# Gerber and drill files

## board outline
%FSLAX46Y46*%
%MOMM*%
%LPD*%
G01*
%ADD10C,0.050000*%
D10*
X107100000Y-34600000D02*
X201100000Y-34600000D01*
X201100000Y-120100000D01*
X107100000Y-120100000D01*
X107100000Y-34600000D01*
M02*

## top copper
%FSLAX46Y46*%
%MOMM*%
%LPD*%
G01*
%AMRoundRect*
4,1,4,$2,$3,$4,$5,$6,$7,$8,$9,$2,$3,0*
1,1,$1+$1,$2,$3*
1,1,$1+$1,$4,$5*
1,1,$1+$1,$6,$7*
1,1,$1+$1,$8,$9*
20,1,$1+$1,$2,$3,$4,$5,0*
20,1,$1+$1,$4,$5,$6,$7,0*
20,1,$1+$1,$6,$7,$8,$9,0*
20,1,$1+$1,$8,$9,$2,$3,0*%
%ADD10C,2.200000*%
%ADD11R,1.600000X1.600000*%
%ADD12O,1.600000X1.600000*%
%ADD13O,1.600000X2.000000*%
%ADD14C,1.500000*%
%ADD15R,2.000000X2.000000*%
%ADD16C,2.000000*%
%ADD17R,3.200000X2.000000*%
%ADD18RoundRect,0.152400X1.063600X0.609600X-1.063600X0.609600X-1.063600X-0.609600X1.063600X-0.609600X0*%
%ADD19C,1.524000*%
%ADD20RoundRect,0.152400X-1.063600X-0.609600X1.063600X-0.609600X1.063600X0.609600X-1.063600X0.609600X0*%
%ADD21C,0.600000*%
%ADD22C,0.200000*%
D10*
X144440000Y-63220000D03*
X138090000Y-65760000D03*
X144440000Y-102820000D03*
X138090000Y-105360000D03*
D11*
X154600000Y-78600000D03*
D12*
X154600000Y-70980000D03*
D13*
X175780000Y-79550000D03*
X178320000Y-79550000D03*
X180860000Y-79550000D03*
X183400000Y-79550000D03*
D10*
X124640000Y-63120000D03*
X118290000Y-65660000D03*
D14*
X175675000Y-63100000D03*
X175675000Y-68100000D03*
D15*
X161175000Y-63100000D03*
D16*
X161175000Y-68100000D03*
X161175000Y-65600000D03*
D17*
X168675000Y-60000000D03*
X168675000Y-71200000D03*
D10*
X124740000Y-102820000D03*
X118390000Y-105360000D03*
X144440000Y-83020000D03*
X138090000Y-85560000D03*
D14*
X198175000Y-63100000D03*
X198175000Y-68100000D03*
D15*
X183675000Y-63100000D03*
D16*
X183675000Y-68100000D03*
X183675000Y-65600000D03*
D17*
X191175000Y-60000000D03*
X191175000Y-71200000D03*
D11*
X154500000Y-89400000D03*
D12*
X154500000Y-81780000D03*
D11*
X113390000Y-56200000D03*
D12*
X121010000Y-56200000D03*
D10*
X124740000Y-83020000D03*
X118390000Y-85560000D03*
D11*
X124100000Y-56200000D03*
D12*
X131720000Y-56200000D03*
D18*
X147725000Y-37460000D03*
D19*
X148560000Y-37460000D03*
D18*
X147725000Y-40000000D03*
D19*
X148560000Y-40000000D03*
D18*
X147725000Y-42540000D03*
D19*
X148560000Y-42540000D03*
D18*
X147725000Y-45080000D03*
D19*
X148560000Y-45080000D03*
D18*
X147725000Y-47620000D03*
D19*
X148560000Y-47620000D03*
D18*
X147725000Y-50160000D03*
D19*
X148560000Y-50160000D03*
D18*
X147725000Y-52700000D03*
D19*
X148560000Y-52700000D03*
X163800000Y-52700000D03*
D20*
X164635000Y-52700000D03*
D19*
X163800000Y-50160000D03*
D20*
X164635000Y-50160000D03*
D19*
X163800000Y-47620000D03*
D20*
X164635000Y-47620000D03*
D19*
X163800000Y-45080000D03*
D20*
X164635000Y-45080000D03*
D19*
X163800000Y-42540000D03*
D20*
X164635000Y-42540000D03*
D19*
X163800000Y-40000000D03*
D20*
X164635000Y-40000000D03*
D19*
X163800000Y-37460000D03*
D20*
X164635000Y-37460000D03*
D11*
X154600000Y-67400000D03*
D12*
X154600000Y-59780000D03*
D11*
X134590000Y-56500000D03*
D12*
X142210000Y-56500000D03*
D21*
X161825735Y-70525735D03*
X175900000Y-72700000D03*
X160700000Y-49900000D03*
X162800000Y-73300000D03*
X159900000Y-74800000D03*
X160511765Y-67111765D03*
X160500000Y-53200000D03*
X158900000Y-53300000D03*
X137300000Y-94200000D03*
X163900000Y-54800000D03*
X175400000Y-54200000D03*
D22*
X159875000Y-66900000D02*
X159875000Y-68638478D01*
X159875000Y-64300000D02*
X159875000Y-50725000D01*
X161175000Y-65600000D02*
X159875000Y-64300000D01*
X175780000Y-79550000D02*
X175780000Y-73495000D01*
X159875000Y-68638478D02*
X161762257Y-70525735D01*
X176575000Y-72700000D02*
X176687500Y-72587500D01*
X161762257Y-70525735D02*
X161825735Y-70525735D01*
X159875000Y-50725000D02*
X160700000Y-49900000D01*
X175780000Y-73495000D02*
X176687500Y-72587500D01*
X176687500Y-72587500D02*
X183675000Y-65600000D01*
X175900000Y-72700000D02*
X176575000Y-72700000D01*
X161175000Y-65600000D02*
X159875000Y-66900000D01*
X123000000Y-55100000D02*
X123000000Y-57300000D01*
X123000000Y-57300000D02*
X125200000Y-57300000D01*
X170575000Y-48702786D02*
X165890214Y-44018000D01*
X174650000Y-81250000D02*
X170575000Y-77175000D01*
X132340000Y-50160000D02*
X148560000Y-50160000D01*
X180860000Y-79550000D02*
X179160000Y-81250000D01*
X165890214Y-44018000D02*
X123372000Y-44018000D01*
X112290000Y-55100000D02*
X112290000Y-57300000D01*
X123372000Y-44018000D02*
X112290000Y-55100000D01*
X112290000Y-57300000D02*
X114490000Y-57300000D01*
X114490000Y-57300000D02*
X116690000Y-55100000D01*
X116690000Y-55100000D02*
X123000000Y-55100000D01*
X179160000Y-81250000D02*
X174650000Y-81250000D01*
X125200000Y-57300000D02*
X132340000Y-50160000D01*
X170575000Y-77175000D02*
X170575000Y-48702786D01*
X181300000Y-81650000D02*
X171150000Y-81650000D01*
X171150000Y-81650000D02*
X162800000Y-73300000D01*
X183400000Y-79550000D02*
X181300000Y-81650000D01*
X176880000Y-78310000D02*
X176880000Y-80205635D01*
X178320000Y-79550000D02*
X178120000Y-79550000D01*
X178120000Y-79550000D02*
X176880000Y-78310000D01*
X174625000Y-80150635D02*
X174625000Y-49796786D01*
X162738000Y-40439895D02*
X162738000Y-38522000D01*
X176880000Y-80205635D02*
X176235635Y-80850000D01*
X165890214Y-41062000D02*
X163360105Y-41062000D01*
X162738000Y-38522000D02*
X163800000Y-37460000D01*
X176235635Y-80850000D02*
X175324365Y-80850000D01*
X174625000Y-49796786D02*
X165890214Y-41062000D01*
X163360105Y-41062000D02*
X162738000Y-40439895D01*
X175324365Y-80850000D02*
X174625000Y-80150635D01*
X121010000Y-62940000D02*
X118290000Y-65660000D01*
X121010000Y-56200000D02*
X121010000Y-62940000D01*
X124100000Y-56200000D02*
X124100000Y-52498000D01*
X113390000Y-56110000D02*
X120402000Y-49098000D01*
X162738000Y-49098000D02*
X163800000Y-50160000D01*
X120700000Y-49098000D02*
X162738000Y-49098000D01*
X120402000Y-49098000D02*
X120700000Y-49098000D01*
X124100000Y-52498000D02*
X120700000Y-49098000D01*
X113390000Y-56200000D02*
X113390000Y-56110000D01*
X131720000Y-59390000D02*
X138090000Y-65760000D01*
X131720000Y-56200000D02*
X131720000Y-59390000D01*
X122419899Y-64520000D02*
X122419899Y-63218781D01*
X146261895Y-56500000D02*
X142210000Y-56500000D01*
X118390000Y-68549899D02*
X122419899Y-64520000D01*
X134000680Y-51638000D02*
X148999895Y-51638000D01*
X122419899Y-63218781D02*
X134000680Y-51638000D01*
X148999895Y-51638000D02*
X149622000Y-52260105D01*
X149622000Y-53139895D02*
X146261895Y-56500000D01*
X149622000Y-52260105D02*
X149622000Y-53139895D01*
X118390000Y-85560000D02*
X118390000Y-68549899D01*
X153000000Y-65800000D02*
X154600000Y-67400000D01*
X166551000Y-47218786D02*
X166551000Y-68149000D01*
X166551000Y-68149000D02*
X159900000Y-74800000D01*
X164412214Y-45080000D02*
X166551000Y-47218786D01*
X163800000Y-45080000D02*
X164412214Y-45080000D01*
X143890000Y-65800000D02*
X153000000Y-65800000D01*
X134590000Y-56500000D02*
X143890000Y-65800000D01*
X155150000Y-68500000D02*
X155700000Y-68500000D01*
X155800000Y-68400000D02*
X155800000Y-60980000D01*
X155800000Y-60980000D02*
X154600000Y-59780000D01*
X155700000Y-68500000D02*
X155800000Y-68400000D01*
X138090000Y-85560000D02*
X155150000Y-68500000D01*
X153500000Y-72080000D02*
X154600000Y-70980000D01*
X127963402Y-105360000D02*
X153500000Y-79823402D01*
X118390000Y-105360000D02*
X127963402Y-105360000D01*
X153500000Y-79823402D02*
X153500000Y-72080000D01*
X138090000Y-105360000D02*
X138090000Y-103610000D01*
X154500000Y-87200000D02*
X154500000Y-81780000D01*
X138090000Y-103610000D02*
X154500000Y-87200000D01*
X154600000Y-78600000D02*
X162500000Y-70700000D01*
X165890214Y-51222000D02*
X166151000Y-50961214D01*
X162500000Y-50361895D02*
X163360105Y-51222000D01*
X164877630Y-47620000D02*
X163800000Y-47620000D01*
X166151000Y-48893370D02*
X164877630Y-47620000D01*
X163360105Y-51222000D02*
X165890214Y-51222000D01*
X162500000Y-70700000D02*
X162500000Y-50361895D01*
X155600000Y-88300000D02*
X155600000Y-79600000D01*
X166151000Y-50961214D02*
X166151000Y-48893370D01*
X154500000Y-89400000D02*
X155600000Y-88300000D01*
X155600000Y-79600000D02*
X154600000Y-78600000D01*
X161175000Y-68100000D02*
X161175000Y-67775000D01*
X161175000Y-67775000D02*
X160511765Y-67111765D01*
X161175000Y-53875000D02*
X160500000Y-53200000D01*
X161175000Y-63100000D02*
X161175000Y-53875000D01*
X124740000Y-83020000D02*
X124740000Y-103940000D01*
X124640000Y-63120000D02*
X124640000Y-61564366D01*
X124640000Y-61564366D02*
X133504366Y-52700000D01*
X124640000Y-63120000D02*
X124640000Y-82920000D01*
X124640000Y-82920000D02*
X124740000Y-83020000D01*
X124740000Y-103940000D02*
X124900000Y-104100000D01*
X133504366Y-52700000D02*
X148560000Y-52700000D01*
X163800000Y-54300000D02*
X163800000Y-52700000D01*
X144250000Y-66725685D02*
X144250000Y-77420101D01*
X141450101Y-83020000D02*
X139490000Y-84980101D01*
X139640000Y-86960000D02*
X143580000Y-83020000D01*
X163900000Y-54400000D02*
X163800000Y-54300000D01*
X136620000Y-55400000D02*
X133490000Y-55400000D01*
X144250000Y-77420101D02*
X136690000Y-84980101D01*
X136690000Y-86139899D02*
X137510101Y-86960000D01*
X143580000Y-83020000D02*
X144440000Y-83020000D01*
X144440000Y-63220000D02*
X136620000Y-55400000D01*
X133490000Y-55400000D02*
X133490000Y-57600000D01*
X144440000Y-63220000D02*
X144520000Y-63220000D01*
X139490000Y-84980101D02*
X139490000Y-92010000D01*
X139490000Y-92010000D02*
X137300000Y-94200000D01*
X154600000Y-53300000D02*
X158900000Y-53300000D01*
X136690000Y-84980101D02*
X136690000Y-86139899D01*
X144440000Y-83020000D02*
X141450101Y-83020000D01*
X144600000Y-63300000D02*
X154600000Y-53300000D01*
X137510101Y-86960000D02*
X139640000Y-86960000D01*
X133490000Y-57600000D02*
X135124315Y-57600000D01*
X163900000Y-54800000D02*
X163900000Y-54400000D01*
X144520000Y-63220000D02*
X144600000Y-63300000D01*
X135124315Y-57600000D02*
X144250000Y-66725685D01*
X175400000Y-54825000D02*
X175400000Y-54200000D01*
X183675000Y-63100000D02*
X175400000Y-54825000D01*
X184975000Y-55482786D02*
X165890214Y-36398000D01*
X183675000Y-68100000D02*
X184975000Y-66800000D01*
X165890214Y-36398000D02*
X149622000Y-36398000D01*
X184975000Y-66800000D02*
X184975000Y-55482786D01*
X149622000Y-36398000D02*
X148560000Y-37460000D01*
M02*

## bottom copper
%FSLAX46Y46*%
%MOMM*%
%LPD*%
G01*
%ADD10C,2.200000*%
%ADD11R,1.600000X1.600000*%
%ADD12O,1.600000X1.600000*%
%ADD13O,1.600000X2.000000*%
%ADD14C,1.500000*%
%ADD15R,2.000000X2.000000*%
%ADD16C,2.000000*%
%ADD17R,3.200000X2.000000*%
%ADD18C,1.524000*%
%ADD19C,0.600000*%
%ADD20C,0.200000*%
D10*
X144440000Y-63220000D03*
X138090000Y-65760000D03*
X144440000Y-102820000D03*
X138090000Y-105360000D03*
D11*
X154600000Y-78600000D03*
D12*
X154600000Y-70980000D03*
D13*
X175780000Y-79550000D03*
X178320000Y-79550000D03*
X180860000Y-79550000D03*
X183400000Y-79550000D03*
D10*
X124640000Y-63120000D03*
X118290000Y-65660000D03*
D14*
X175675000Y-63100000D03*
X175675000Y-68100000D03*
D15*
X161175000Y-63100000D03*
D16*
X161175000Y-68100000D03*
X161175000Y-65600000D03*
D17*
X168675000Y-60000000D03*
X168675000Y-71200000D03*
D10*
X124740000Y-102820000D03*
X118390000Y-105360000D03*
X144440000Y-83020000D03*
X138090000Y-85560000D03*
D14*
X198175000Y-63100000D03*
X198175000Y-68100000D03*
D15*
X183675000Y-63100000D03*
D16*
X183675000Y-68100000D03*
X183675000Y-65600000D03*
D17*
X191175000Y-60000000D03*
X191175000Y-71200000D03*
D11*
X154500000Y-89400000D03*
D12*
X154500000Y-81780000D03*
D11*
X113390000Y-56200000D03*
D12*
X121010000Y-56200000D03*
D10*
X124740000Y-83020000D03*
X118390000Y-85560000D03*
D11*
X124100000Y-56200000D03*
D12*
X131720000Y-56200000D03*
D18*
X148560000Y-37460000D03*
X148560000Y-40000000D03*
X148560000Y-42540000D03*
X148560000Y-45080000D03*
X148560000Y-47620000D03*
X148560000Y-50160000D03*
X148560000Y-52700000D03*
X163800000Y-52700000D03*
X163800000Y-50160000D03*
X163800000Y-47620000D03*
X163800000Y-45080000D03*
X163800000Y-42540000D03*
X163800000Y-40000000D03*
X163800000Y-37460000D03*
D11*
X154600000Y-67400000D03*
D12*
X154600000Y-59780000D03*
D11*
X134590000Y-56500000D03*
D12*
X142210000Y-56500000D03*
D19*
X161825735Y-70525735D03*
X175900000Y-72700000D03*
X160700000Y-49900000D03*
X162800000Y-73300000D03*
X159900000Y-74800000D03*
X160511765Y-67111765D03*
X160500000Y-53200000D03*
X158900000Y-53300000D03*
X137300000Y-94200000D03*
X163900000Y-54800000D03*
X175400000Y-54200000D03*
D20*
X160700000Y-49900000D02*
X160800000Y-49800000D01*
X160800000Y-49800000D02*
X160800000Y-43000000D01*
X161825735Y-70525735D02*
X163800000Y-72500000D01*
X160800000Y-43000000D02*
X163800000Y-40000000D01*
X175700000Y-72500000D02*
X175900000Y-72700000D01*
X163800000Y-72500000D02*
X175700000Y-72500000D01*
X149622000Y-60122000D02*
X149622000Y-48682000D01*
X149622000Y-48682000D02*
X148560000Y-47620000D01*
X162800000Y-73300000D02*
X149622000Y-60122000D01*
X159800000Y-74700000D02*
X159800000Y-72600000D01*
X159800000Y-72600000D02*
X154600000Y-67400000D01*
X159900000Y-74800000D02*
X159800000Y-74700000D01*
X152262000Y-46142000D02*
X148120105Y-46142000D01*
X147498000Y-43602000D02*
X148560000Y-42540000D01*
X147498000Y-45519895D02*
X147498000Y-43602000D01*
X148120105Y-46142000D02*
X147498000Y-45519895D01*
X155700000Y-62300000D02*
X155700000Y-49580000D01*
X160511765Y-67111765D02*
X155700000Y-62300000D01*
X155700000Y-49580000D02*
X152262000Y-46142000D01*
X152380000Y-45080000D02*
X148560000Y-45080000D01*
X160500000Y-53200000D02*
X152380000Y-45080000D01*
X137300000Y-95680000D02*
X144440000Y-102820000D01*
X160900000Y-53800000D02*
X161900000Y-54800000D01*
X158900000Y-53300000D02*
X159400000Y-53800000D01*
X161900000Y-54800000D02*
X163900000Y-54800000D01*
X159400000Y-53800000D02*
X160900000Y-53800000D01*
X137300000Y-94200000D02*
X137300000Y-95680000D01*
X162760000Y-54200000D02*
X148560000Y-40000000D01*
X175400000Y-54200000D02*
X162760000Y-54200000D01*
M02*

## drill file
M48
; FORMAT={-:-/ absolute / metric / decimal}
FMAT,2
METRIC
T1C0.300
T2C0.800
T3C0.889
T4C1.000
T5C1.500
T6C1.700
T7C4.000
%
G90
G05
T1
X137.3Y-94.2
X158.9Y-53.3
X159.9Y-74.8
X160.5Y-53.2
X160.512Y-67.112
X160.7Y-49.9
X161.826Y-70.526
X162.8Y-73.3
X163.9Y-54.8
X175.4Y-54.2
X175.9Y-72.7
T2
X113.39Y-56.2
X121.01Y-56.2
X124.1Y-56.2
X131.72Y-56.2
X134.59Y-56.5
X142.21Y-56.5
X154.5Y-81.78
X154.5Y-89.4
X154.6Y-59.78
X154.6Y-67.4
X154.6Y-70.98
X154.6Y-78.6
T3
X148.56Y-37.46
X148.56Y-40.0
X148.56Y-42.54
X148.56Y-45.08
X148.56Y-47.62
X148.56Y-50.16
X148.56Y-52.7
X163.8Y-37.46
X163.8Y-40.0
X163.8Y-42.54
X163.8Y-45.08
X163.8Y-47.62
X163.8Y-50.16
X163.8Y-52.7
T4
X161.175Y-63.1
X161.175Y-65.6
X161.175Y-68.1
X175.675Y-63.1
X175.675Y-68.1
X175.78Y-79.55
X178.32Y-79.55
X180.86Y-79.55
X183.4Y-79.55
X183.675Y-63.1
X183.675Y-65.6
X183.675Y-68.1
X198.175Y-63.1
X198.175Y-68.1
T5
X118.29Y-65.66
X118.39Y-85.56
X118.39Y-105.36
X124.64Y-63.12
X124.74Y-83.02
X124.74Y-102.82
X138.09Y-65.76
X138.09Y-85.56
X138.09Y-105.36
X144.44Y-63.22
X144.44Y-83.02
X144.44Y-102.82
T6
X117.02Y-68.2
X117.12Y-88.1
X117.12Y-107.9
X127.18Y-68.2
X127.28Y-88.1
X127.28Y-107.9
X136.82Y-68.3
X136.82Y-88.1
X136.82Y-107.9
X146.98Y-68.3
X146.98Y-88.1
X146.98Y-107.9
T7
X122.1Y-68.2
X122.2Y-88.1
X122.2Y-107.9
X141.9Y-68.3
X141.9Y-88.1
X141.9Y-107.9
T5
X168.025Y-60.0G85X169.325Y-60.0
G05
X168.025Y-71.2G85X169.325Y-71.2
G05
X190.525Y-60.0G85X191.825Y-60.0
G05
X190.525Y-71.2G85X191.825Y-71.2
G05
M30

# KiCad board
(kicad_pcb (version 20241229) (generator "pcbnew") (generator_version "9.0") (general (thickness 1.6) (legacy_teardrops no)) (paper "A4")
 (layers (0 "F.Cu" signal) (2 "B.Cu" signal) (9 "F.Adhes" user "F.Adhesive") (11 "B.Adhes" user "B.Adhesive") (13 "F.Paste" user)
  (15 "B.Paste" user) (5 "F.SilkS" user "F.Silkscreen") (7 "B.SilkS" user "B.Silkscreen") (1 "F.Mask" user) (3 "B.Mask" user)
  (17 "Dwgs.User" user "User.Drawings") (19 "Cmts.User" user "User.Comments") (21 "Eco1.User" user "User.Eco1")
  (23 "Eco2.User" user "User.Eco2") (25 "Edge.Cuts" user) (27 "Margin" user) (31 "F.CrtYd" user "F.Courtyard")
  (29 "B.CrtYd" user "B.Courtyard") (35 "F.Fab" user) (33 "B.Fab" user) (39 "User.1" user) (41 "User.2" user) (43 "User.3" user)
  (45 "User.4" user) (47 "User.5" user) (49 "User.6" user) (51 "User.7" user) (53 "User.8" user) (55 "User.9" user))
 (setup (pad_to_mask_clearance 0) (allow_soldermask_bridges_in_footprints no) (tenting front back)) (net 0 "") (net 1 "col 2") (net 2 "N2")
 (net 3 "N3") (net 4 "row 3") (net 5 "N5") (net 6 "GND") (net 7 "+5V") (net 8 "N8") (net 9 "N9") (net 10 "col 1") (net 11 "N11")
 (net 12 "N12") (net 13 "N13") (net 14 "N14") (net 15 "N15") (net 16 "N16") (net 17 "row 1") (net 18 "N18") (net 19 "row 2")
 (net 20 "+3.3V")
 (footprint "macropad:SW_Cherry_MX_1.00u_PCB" (layer "F.Cu") (at 144.44 63.22)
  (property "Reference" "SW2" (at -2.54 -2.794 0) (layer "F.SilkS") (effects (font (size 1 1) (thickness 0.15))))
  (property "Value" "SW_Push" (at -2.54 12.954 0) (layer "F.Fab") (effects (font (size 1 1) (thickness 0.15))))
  (pad "" np_thru_hole circle (at -7.62 5.08) (size 1.7 1.7) (drill 1.7) (layers "*.Cu" "*.Mask"))
  (pad "" np_thru_hole circle (at -2.54 5.08) (size 4 4) (drill 4) (layers "*.Cu" "*.Mask"))
  (pad "" np_thru_hole circle (at 2.54 5.08) (size 1.7 1.7) (drill 1.7) (layers "*.Cu" "*.Mask"))
  (pad "1" thru_hole circle (at 0 0) (size 2.2 2.2) (drill 1.5) (layers "*.Cu" "*.Mask") (remove_unused_layers no) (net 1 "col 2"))
  (pad "2" thru_hole circle (at -6.35 2.54) (size 2.2 2.2) (drill 1.5) (layers "*.Cu" "*.Mask") (remove_unused_layers no) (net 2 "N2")))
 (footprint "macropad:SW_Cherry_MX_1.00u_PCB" (layer "F.Cu") (at 144.44 102.82)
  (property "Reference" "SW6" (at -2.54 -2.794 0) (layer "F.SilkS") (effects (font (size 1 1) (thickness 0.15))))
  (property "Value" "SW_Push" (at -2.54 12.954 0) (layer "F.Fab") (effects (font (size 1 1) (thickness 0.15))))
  (pad "" np_thru_hole circle (at -7.62 5.08) (size 1.7 1.7) (drill 1.7) (layers "*.Cu" "*.Mask"))
  (pad "" np_thru_hole circle (at -2.54 5.08) (size 4 4) (drill 4) (layers "*.Cu" "*.Mask"))
  (pad "" np_thru_hole circle (at 2.54 5.08) (size 1.7 1.7) (drill 1.7) (layers "*.Cu" "*.Mask"))
  (pad "1" thru_hole circle (at 0 0) (size 2.2 2.2) (drill 1.5) (layers "*.Cu" "*.Mask") (remove_unused_layers no) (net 1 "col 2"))
  (pad "2" thru_hole circle (at -6.35 2.54) (size 2.2 2.2) (drill 1.5) (layers "*.Cu" "*.Mask") (remove_unused_layers no) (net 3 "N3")))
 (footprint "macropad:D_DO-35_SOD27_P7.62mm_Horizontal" (layer "F.Cu") (at 154.6 78.6 90)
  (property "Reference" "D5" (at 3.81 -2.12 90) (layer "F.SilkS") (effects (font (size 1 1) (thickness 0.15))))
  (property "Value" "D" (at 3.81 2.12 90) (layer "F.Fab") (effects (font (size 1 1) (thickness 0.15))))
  (pad "1" thru_hole rect (at 0 0 90) (size 1.6 1.6) (drill 0.8) (layers "*.Cu" "*.Mask") (remove_unused_layers no) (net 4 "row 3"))
  (pad "2" thru_hole oval (at 7.62 0 90) (size 1.6 1.6) (drill 0.8) (layers "*.Cu" "*.Mask") (remove_unused_layers no) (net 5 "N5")))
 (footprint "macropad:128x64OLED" (layer "F.Cu") (at 179.4 90.15)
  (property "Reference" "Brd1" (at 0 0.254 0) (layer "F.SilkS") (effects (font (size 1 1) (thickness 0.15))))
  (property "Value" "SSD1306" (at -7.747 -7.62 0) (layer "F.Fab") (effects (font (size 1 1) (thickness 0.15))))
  (pad "1" thru_hole oval (at -3.62 -10.6 90) (size 2 1.6) (drill 1) (layers "*.Cu" "*.Mask") (remove_unused_layers no) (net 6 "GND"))
  (pad "2" thru_hole oval (at -1.08 -10.6 90) (size 2 1.6) (drill 1) (layers "*.Cu" "*.Mask") (remove_unused_layers no) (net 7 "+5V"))
  (pad "3" thru_hole oval (at 1.46 -10.6 90) (size 2 1.6) (drill 1) (layers "*.Cu" "*.Mask") (remove_unused_layers no) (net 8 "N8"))
  (pad "4" thru_hole oval (at 4 -10.6 90) (size 2 1.6) (drill 1) (layers "*.Cu" "*.Mask") (remove_unused_layers no) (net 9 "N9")))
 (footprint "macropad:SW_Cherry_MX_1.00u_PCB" (layer "F.Cu") (at 124.64 63.12)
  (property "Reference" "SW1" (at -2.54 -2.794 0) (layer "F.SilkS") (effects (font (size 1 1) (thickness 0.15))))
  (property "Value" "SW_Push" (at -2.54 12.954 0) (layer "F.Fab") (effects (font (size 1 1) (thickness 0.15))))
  (pad "" np_thru_hole circle (at -7.62 5.08) (size 1.7 1.7) (drill 1.7) (layers "*.Cu" "*.Mask"))
  (pad "" np_thru_hole circle (at -2.54 5.08) (size 4 4) (drill 4) (layers "*.Cu" "*.Mask"))
  (pad "" np_thru_hole circle (at 2.54 5.08) (size 1.7 1.7) (drill 1.7) (layers "*.Cu" "*.Mask"))
  (pad "1" thru_hole circle (at 0 0) (size 2.2 2.2) (drill 1.5) (layers "*.Cu" "*.Mask") (remove_unused_layers no) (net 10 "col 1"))
  (pad "2" thru_hole circle (at -6.35 2.54) (size 2.2 2.2) (drill 1.5) (layers "*.Cu" "*.Mask") (remove_unused_layers no) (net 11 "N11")))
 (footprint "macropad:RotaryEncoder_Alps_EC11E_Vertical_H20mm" (layer "F.Cu") (at 161.175 63.1)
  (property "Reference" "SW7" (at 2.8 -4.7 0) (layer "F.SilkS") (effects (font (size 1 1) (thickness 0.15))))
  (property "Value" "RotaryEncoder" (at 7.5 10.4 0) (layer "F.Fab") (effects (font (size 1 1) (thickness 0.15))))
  (pad "" thru_hole circle (at 14.5 0) (size 1.5 1.5) (drill 1) (layers "*.Cu" "*.Mask") (remove_unused_layers no))
  (pad "" thru_hole circle (at 14.5 5) (size 1.5 1.5) (drill 1) (layers "*.Cu" "*.Mask") (remove_unused_layers no))
  (pad "A" thru_hole rect (at 0 0) (size 2 2) (drill 1) (layers "*.Cu" "*.Mask") (remove_unused_layers no) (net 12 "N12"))
  (pad "B" thru_hole circle (at 0 5) (size 2 2) (drill 1) (layers "*.Cu" "*.Mask") (remove_unused_layers no) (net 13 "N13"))
  (pad "C" thru_hole circle (at 0 2.5) (size 2 2) (drill 1) (layers "*.Cu" "*.Mask") (remove_unused_layers no) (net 6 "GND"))
  (pad "MP" thru_hole rect (at 7.5 -3.1) (size 3.2 2) (drill oval 2.8 1.5) (layers "*.Cu" "*.Mask") (remove_unused_layers no))
  (pad "MP" thru_hole rect (at 7.5 8.1) (size 3.2 2) (drill oval 2.8 1.5) (layers "*.Cu" "*.Mask") (remove_unused_layers no)))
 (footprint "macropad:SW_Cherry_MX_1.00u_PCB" (layer "F.Cu") (at 124.74 102.82)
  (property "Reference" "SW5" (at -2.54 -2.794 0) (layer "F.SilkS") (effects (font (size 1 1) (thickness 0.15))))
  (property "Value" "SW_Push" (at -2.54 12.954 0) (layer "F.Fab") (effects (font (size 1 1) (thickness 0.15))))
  (pad "" np_thru_hole circle (at -7.62 5.08) (size 1.7 1.7) (drill 1.7) (layers "*.Cu" "*.Mask"))
  (pad "" np_thru_hole circle (at -2.54 5.08) (size 4 4) (drill 4) (layers "*.Cu" "*.Mask"))
  (pad "" np_thru_hole circle (at 2.54 5.08) (size 1.7 1.7) (drill 1.7) (layers "*.Cu" "*.Mask"))
  (pad "1" thru_hole circle (at 0 0) (size 2.2 2.2) (drill 1.5) (layers "*.Cu" "*.Mask") (remove_unused_layers no) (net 10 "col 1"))
  (pad "2" thru_hole circle (at -6.35 2.54) (size 2.2 2.2) (drill 1.5) (layers "*.Cu" "*.Mask") (remove_unused_layers no) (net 5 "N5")))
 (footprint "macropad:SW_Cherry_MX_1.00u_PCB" (layer "F.Cu") (at 144.44 83.02)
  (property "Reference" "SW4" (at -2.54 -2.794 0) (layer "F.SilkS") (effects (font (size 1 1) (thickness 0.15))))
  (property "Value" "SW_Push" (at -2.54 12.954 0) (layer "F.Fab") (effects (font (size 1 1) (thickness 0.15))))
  (pad "" np_thru_hole circle (at -7.62 5.08) (size 1.7 1.7) (drill 1.7) (layers "*.Cu" "*.Mask"))
  (pad "" np_thru_hole circle (at -2.54 5.08) (size 4 4) (drill 4) (layers "*.Cu" "*.Mask"))
  (pad "" np_thru_hole circle (at 2.54 5.08) (size 1.7 1.7) (drill 1.7) (layers "*.Cu" "*.Mask"))
  (pad "1" thru_hole circle (at 0 0) (size 2.2 2.2) (drill 1.5) (layers "*.Cu" "*.Mask") (remove_unused_layers no) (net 1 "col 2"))
  (pad "2" thru_hole circle (at -6.35 2.54) (size 2.2 2.2) (drill 1.5) (layers "*.Cu" "*.Mask") (remove_unused_layers no) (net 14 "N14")))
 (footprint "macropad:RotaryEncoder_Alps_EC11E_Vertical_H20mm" (layer "F.Cu") (at 183.675 63.1)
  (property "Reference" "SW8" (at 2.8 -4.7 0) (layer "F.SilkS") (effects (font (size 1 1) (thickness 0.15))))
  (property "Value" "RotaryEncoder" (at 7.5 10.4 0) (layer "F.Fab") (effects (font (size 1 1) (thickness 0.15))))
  (pad "" thru_hole circle (at 14.5 0) (size 1.5 1.5) (drill 1) (layers "*.Cu" "*.Mask") (remove_unused_layers no))
  (pad "" thru_hole circle (at 14.5 5) (size 1.5 1.5) (drill 1) (layers "*.Cu" "*.Mask") (remove_unused_layers no))
  (pad "A" thru_hole rect (at 0 0) (size 2 2) (drill 1) (layers "*.Cu" "*.Mask") (remove_unused_layers no) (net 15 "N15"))
  (pad "B" thru_hole circle (at 0 5) (size 2 2) (drill 1) (layers "*.Cu" "*.Mask") (remove_unused_layers no) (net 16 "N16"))
  (pad "C" thru_hole circle (at 0 2.5) (size 2 2) (drill 1) (layers "*.Cu" "*.Mask") (remove_unused_layers no) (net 6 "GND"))
  (pad "MP" thru_hole rect (at 7.5 -3.1) (size 3.2 2) (drill oval 2.8 1.5) (layers "*.Cu" "*.Mask") (remove_unused_layers no))
  (pad "MP" thru_hole rect (at 7.5 8.1) (size 3.2 2) (drill oval 2.8 1.5) (layers "*.Cu" "*.Mask") (remove_unused_layers no)))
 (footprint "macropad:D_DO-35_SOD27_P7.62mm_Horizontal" (layer "F.Cu") (at 154.5 89.4 90)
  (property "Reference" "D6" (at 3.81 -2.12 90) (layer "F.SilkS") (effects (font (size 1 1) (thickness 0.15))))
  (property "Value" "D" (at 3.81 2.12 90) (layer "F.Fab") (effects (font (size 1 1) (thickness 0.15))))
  (pad "1" thru_hole rect (at 0 0 90) (size 1.6 1.6) (drill 0.8) (layers "*.Cu" "*.Mask") (remove_unused_layers no) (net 4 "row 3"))
  (pad "2" thru_hole oval (at 7.62 0 90) (size 1.6 1.6) (drill 0.8) (layers "*.Cu" "*.Mask") (remove_unused_layers no) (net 3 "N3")))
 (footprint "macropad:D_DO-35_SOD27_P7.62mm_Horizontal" (layer "F.Cu") (at 113.39 56.2)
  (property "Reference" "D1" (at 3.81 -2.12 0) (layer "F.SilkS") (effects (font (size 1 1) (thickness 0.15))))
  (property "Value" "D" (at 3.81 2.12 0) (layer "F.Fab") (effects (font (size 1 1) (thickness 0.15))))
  (pad "1" thru_hole rect (at 0 0) (size 1.6 1.6) (drill 0.8) (layers "*.Cu" "*.Mask") (remove_unused_layers no) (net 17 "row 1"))
  (pad "2" thru_hole oval (at 7.62 0) (size 1.6 1.6) (drill 0.8) (layers "*.Cu" "*.Mask") (remove_unused_layers no) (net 11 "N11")))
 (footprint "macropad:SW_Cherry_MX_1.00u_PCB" (layer "F.Cu") (at 124.74 83.02)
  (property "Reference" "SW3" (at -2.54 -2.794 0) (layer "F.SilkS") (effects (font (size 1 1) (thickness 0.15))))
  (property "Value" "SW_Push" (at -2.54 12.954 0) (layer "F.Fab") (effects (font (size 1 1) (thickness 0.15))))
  (pad "" np_thru_hole circle (at -7.62 5.08) (size 1.7 1.7) (drill 1.7) (layers "*.Cu" "*.Mask"))
  (pad "" np_thru_hole circle (at -2.54 5.08) (size 4 4) (drill 4) (layers "*.Cu" "*.Mask"))
  (pad "" np_thru_hole circle (at 2.54 5.08) (size 1.7 1.7) (drill 1.7) (layers "*.Cu" "*.Mask"))
  (pad "1" thru_hole circle (at 0 0) (size 2.2 2.2) (drill 1.5) (layers "*.Cu" "*.Mask") (remove_unused_layers no) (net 10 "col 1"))
  (pad "2" thru_hole circle (at -6.35 2.54) (size 2.2 2.2) (drill 1.5) (layers "*.Cu" "*.Mask") (remove_unused_layers no) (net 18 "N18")))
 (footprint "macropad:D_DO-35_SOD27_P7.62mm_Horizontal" (layer "F.Cu") (at 124.1 56.2)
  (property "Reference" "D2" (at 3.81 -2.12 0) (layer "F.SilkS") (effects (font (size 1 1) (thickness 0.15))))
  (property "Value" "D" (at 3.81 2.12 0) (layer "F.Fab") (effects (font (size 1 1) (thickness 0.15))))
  (pad "1" thru_hole rect (at 0 0) (size 1.6 1.6) (drill 0.8) (layers "*.Cu" "*.Mask") (remove_unused_layers no) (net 17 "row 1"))
  (pad "2" thru_hole oval (at 7.62 0) (size 1.6 1.6) (drill 0.8) (layers "*.Cu" "*.Mask") (remove_unused_layers no) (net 2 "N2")))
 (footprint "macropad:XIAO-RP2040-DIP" (layer "F.Cu") (at 156.18 45.08)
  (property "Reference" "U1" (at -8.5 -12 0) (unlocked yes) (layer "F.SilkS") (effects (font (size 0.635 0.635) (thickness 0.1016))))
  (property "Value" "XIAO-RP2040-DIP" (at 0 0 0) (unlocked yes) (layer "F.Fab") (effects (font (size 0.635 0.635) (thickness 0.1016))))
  (pad "1" smd roundrect (at -8.455 -7.62 180) (size 2.432 1.524) (layers "F.Cu" "F.Mask") (roundrect_rratio 0.1) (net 16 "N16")
   (thermal_bridge_angle 45))
  (pad "1" thru_hole circle (at -7.62 -7.62 180) (size 1.524 1.524) (drill 0.889) (layers "*.Cu" "*.Mask") (remove_unused_layers no)
   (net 16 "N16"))
  (pad "2" smd roundrect (at -8.455 -5.08 180) (size 2.432 1.524) (layers "F.Cu" "F.Mask") (roundrect_rratio 0.1) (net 15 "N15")
   (thermal_bridge_angle 45))
  (pad "2" thru_hole circle (at -7.62 -5.08 180) (size 1.524 1.524) (drill 0.889) (layers "*.Cu" "*.Mask") (remove_unused_layers no)
   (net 15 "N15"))
  (pad "3" smd roundrect (at -8.455 -2.54 180) (size 2.432 1.524) (layers "F.Cu" "F.Mask") (roundrect_rratio 0.1) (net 13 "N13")
   (thermal_bridge_angle 45))
  (pad "3" thru_hole circle (at -7.62 -2.54 180) (size 1.524 1.524) (drill 0.889) (layers "*.Cu" "*.Mask") (remove_unused_layers no)
   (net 13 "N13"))
  (pad "4" smd roundrect (at -8.455 0 180) (size 2.432 1.524) (layers "F.Cu" "F.Mask") (roundrect_rratio 0.1) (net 12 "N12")
   (thermal_bridge_angle 45))
  (pad "4" thru_hole circle (at -7.62 0 180) (size 1.524 1.524) (drill 0.889) (layers "*.Cu" "*.Mask") (remove_unused_layers no)
   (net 12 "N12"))
  (pad "5" smd roundrect (at -8.455 2.54 180) (size 2.432 1.524) (layers "F.Cu" "F.Mask") (roundrect_rratio 0.1) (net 9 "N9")
   (thermal_bridge_angle 45))
  (pad "5" thru_hole circle (at -7.62 2.54 180) (size 1.524 1.524) (drill 0.889) (layers "*.Cu" "*.Mask") (remove_unused_layers no)
   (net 9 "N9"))
  (pad "6" smd roundrect (at -8.455 5.08 180) (size 2.432 1.524) (layers "F.Cu" "F.Mask") (roundrect_rratio 0.1) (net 8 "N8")
   (thermal_bridge_angle 45))
  (pad "6" thru_hole circle (at -7.62 5.08 180) (size 1.524 1.524) (drill 0.889) (layers "*.Cu" "*.Mask") (remove_unused_layers no)
   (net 8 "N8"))
  (pad "7" smd roundrect (at -8.455 7.62 180) (size 2.432 1.524) (layers "F.Cu" "F.Mask") (roundrect_rratio 0.1) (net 10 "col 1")
   (thermal_bridge_angle 45))
  (pad "7" thru_hole circle (at -7.62 7.62 180) (size 1.524 1.524) (drill 0.889) (layers "*.Cu" "*.Mask") (remove_unused_layers no)
   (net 10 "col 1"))
  (pad "8" thru_hole circle (at 7.62 7.62) (size 1.524 1.524) (drill 0.889) (layers "*.Cu" "*.Mask") (remove_unused_layers no)
   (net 1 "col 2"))
  (pad "8" smd roundrect (at 8.455 7.62) (size 2.432 1.524) (layers "F.Cu" "F.Mask") (roundrect_rratio 0.1) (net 1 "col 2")
   (thermal_bridge_angle 45))
  (pad "9" thru_hole circle (at 7.62 5.08) (size 1.524 1.524) (drill 0.889) (layers "*.Cu" "*.Mask") (remove_unused_layers no)
   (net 17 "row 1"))
  (pad "9" smd roundrect (at 8.455 5.08) (size 2.432 1.524) (layers "F.Cu" "F.Mask") (roundrect_rratio 0.1) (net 17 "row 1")
   (thermal_bridge_angle 45))
  (pad "10" thru_hole circle (at 7.62 2.54) (size 1.524 1.524) (drill 0.889) (layers "*.Cu" "*.Mask") (remove_unused_layers no)
   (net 4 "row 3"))
  (pad "10" smd roundrect (at 8.455 2.54) (size 2.432 1.524) (layers "F.Cu" "F.Mask") (roundrect_rratio 0.1) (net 4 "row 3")
   (thermal_bridge_angle 45))
  (pad "11" thru_hole circle (at 7.62 0) (size 1.524 1.524) (drill 0.889) (layers "*.Cu" "*.Mask") (remove_unused_layers no)
   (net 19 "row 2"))
  (pad "11" smd roundrect (at 8.455 0) (size 2.432 1.524) (layers "F.Cu" "F.Mask") (roundrect_rratio 0.1) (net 19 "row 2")
   (thermal_bridge_angle 45))
  (pad "12" thru_hole circle (at 7.62 -2.54) (size 1.524 1.524) (drill 0.889) (layers "*.Cu" "*.Mask") (remove_unused_layers no)
   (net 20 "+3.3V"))
  (pad "12" smd roundrect (at 8.455 -2.54) (size 2.432 1.524) (layers "F.Cu" "F.Mask") (roundrect_rratio 0.1) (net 20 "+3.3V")
   (thermal_bridge_angle 45))
  (pad "13" thru_hole circle (at 7.62 -5.08) (size 1.524 1.524) (drill 0.889) (layers "*.Cu" "*.Mask") (remove_unused_layers no)
   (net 6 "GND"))
  (pad "13" smd roundrect (at 8.455 -5.08) (size 2.432 1.524) (layers "F.Cu" "F.Mask") (roundrect_rratio 0.1) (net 6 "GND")
   (thermal_bridge_angle 45))
  (pad "14" thru_hole circle (at 7.62 -7.62) (size 1.524 1.524) (drill 0.889) (layers "*.Cu" "*.Mask") (remove_unused_layers no)
   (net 7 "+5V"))
  (pad "14" smd roundrect (at 8.455 -7.62) (size 2.432 1.524) (layers "F.Cu" "F.Mask") (roundrect_rratio 0.1) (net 7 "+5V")
   (thermal_bridge_angle 45)))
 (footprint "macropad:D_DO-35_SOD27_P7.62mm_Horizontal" (layer "F.Cu") (at 154.6 67.4 90)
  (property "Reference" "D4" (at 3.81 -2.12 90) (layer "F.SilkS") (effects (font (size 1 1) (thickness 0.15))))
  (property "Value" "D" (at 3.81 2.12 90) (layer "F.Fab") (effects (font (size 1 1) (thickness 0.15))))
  (pad "1" thru_hole rect (at 0 0 90) (size 1.6 1.6) (drill 0.8) (layers "*.Cu" "*.Mask") (remove_unused_layers no) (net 19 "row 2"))
  (pad "2" thru_hole oval (at 7.62 0 90) (size 1.6 1.6) (drill 0.8) (layers "*.Cu" "*.Mask") (remove_unused_layers no) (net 14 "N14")))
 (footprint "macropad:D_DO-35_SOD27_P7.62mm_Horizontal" (layer "F.Cu") (at 134.59 56.5)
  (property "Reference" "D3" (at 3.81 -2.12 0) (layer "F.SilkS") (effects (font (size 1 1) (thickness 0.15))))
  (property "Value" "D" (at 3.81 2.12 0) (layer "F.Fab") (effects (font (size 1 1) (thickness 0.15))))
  (pad "1" thru_hole rect (at 0 0) (size 1.6 1.6) (drill 0.8) (layers "*.Cu" "*.Mask") (remove_unused_layers no) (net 19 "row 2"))
  (pad "2" thru_hole oval (at 7.62 0) (size 1.6 1.6) (drill 0.8) (layers "*.Cu" "*.Mask") (remove_unused_layers no) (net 18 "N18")))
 (gr_rect (start 107.1 34.6) (end 201.1 120.1) (stroke (width 0.05) (type default)) (fill no) (layer "Edge.Cuts"))
 (segment (start 159.875 66.9) (end 159.875 68.638478) (width 0.2) (layer "F.Cu") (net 6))
 (segment (start 159.875 64.3) (end 159.875 50.725) (width 0.2) (layer "F.Cu") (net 6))
 (segment (start 161.175 65.6) (end 159.875 64.3) (width 0.2) (layer "F.Cu") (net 6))
 (segment (start 175.78 79.55) (end 175.78 73.495) (width 0.2) (layer "F.Cu") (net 6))
 (segment (start 159.875 68.638478) (end 161.762257 70.525735) (width 0.2) (layer "F.Cu") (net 6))
 (segment (start 176.575 72.7) (end 176.6875 72.5875) (width 0.2) (layer "F.Cu") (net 6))
 (segment (start 161.762257 70.525735) (end 161.825735 70.525735) (width 0.2) (layer "F.Cu") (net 6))
 (segment (start 159.875 50.725) (end 160.7 49.9) (width 0.2) (layer "F.Cu") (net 6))
 (segment (start 175.78 73.495) (end 176.6875 72.5875) (width 0.2) (layer "F.Cu") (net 6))
 (segment (start 176.6875 72.5875) (end 183.675 65.6) (width 0.2) (layer "F.Cu") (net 6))
 (segment (start 175.9 72.7) (end 176.575 72.7) (width 0.2) (layer "F.Cu") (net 6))
 (segment (start 161.175 65.6) (end 159.875 66.9) (width 0.2) (layer "F.Cu") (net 6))
 (via (at 161.825735 70.525735) (size 0.6) (drill 0.3) (layers "F.Cu" "B.Cu") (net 6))
 (via (at 175.9 72.7) (size 0.6) (drill 0.3) (layers "F.Cu" "B.Cu") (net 6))
 (via (at 160.7 49.9) (size 0.6) (drill 0.3) (layers "F.Cu" "B.Cu") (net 6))
 (segment (start 160.7 49.9) (end 160.8 49.8) (width 0.2) (layer "B.Cu") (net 6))
 (segment (start 160.8 49.8) (end 160.8 43) (width 0.2) (layer "B.Cu") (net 6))
 (segment (start 161.825735 70.525735) (end 163.8 72.5) (width 0.2) (layer "B.Cu") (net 6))
 (segment (start 160.8 43) (end 163.8 40) (width 0.2) (layer "B.Cu") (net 6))
 (segment (start 175.7 72.5) (end 175.9 72.7) (width 0.2) (layer "B.Cu") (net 6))
 (segment (start 163.8 72.5) (end 175.7 72.5) (width 0.2) (layer "B.Cu") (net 6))
 (segment (start 123 55.1) (end 123 57.3) (width 0.2) (layer "F.Cu") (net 8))
 (segment (start 123 57.3) (end 125.2 57.3) (width 0.2) (layer "F.Cu") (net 8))
 (segment (start 170.575 48.702786) (end 165.890214 44.018) (width 0.2) (layer "F.Cu") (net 8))
 (segment (start 174.65 81.25) (end 170.575 77.175) (width 0.2) (layer "F.Cu") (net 8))
 (segment (start 132.34 50.16) (end 148.56 50.16) (width 0.2) (layer "F.Cu") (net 8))
 (segment (start 180.86 79.55) (end 179.16 81.25) (width 0.2) (layer "F.Cu") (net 8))
 (segment (start 165.890214 44.018) (end 123.372 44.018) (width 0.2) (layer "F.Cu") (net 8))
 (segment (start 112.29 55.1) (end 112.29 57.3) (width 0.2) (layer "F.Cu") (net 8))
 (segment (start 123.372 44.018) (end 112.29 55.1) (width 0.2) (layer "F.Cu") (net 8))
 (segment (start 112.29 57.3) (end 114.49 57.3) (width 0.2) (layer "F.Cu") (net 8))
 (segment (start 114.49 57.3) (end 116.69 55.1) (width 0.2) (layer "F.Cu") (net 8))
 (segment (start 116.69 55.1) (end 123 55.1) (width 0.2) (layer "F.Cu") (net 8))
 (segment (start 179.16 81.25) (end 174.65 81.25) (width 0.2) (layer "F.Cu") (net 8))
 (segment (start 125.2 57.3) (end 132.34 50.16) (width 0.2) (layer "F.Cu") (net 8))
 (segment (start 170.575 77.175) (end 170.575 48.702786) (width 0.2) (layer "F.Cu") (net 8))
 (segment (start 181.3 81.65) (end 171.15 81.65) (width 0.2) (layer "F.Cu") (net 9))
 (segment (start 171.15 81.65) (end 162.8 73.3) (width 0.2) (layer "F.Cu") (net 9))
 (segment (start 183.4 79.55) (end 181.3 81.65) (width 0.2) (layer "F.Cu") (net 9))
 (via (at 162.8 73.3) (size 0.6) (drill 0.3) (layers "F.Cu" "B.Cu") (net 9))
 (segment (start 149.622 60.122) (end 149.622 48.682) (width 0.2) (layer "B.Cu") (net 9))
 (segment (start 149.622 48.682) (end 148.56 47.62) (width 0.2) (layer "B.Cu") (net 9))
 (segment (start 162.8 73.3) (end 149.622 60.122) (width 0.2) (layer "B.Cu") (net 9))
 (segment (start 176.88 78.31) (end 176.88 80.205635) (width 0.2) (layer "F.Cu") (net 7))
 (segment (start 178.32 79.55) (end 178.12 79.55) (width 0.2) (layer "F.Cu") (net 7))
 (segment (start 178.12 79.55) (end 176.88 78.31) (width 0.2) (layer "F.Cu") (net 7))
 (segment (start 174.625 80.150635) (end 174.625 49.796786) (width 0.2) (layer "F.Cu") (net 7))
 (segment (start 162.738 40.439895) (end 162.738 38.522) (width 0.2) (layer "F.Cu") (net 7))
 (segment (start 176.88 80.205635) (end 176.235635 80.85) (width 0.2) (layer "F.Cu") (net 7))
 (segment (start 165.890214 41.062) (end 163.360105 41.062) (width 0.2) (layer "F.Cu") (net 7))
 (segment (start 162.738 38.522) (end 163.8 37.46) (width 0.2) (layer "F.Cu") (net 7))
 (segment (start 176.235635 80.85) (end 175.324365 80.85) (width 0.2) (layer "F.Cu") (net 7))
 (segment (start 174.625 49.796786) (end 165.890214 41.062) (width 0.2) (layer "F.Cu") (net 7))
 (segment (start 163.360105 41.062) (end 162.738 40.439895) (width 0.2) (layer "F.Cu") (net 7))
 (segment (start 175.324365 80.85) (end 174.625 80.150635) (width 0.2) (layer "F.Cu") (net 7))
 (segment (start 121.01 62.94) (end 118.29 65.66) (width 0.2) (layer "F.Cu") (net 11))
 (segment (start 121.01 56.2) (end 121.01 62.94) (width 0.2) (layer "F.Cu") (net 11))
 (segment (start 124.1 56.2) (end 124.1 52.498) (width 0.2) (layer "F.Cu") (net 17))
 (segment (start 113.39 56.11) (end 120.402 49.098) (width 0.2) (layer "F.Cu") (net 17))
 (segment (start 162.738 49.098) (end 163.8 50.16) (width 0.2) (layer "F.Cu") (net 17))
 (segment (start 120.7 49.098) (end 162.738 49.098) (width 0.2) (layer "F.Cu") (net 17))
 (segment (start 120.402 49.098) (end 120.7 49.098) (width 0.2) (layer "F.Cu") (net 17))
 (segment (start 124.1 52.498) (end 120.7 49.098) (width 0.2) (layer "F.Cu") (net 17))
 (segment (start 113.39 56.2) (end 113.39 56.11) (width 0.2) (layer "F.Cu") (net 17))
 (segment (start 131.72 59.39) (end 138.09 65.76) (width 0.2) (layer "F.Cu") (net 2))
 (segment (start 131.72 56.2) (end 131.72 59.39) (width 0.2) (layer "F.Cu") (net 2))
 (segment (start 122.419899 64.52) (end 122.419899 63.218781) (width 0.2) (layer "F.Cu") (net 18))
 (segment (start 146.261895 56.5) (end 142.21 56.5) (width 0.2) (layer "F.Cu") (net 18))
 (segment (start 118.39 68.549899) (end 122.419899 64.52) (width 0.2) (layer "F.Cu") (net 18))
 (segment (start 134.00068 51.638) (end 148.999895 51.638) (width 0.2) (layer "F.Cu") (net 18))
 (segment (start 122.419899 63.218781) (end 134.00068 51.638) (width 0.2) (layer "F.Cu") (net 18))
 (segment (start 148.999895 51.638) (end 149.622 52.260105) (width 0.2) (layer "F.Cu") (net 18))
 (segment (start 149.622 53.139895) (end 146.261895 56.5) (width 0.2) (layer "F.Cu") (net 18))
 (segment (start 149.622 52.260105) (end 149.622 53.139895) (width 0.2) (layer "F.Cu") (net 18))
 (segment (start 118.39 85.56) (end 118.39 68.549899) (width 0.2) (layer "F.Cu") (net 18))
 (segment (start 153 65.8) (end 154.6 67.4) (width 0.2) (layer "F.Cu") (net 19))
 (segment (start 166.551 47.218786) (end 166.551 68.149) (width 0.2) (layer "F.Cu") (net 19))
 (segment (start 166.551 68.149) (end 159.9 74.8) (width 0.2) (layer "F.Cu") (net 19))
 (segment (start 164.412214 45.08) (end 166.551 47.218786) (width 0.2) (layer "F.Cu") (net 19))
 (segment (start 163.8 45.08) (end 164.412214 45.08) (width 0.2) (layer "F.Cu") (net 19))
 (segment (start 143.89 65.8) (end 153 65.8) (width 0.2) (layer "F.Cu") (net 19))
 (segment (start 134.59 56.5) (end 143.89 65.8) (width 0.2) (layer "F.Cu") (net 19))
 (via (at 159.9 74.8) (size 0.6) (drill 0.3) (layers "F.Cu" "B.Cu") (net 19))
 (segment (start 159.8 74.7) (end 159.8 72.6) (width 0.2) (layer "B.Cu") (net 19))
 (segment (start 159.8 72.6) (end 154.6 67.4) (width 0.2) (layer "B.Cu") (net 19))
 (segment (start 159.9 74.8) (end 159.8 74.7) (width 0.2) (layer "B.Cu") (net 19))
 (segment (start 155.15 68.5) (end 155.7 68.5) (width 0.2) (layer "F.Cu") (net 14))
 (segment (start 155.8 68.4) (end 155.8 60.98) (width 0.2) (layer "F.Cu") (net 14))
 (segment (start 155.8 60.98) (end 154.6 59.78) (width 0.2) (layer "F.Cu") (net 14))
 (segment (start 155.7 68.5) (end 155.8 68.4) (width 0.2) (layer "F.Cu") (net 14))
 (segment (start 138.09 85.56) (end 155.15 68.5) (width 0.2) (layer "F.Cu") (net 14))
 (segment (start 153.5 72.08) (end 154.6 70.98) (width 0.2) (layer "F.Cu") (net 5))
 (segment (start 127.963402 105.36) (end 153.5 79.823402) (width 0.2) (layer "F.Cu") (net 5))
 (segment (start 118.39 105.36) (end 127.963402 105.36) (width 0.2) (layer "F.Cu") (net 5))
 (segment (start 153.5 79.823402) (end 153.5 72.08) (width 0.2) (layer "F.Cu") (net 5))
 (segment (start 138.09 105.36) (end 138.09 103.61) (width 0.2) (layer "F.Cu") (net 3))
 (segment (start 154.5 87.2) (end 154.5 81.78) (width 0.2) (layer "F.Cu") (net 3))
 (segment (start 138.09 103.61) (end 154.5 87.2) (width 0.2) (layer "F.Cu") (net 3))
 (segment (start 154.6 78.6) (end 162.5 70.7) (width 0.2) (layer "F.Cu") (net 4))
 (segment (start 165.890214 51.222) (end 166.151 50.961214) (width 0.2) (layer "F.Cu") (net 4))
 (segment (start 162.5 50.361895) (end 163.360105 51.222) (width 0.2) (layer "F.Cu") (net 4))
 (segment (start 164.87763 47.62) (end 163.8 47.62) (width 0.2) (layer "F.Cu") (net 4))
 (segment (start 166.151 48.89337) (end 164.87763 47.62) (width 0.2) (layer "F.Cu") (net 4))
 (segment (start 163.360105 51.222) (end 165.890214 51.222) (width 0.2) (layer "F.Cu") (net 4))
 (segment (start 162.5 70.7) (end 162.5 50.361895) (width 0.2) (layer "F.Cu") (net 4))
 (segment (start 155.6 88.3) (end 155.6 79.6) (width 0.2) (layer "F.Cu") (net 4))
 (segment (start 166.151 50.961214) (end 166.151 48.89337) (width 0.2) (layer "F.Cu") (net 4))
 (segment (start 154.5 89.4) (end 155.6 88.3) (width 0.2) (layer "F.Cu") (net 4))
 (segment (start 155.6 79.6) (end 154.6 78.6) (width 0.2) (layer "F.Cu") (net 4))
 (segment (start 161.175 68.1) (end 161.175 67.775) (width 0.2) (layer "F.Cu") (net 13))
 (segment (start 161.175 67.775) (end 160.511765 67.111765) (width 0.2) (layer "F.Cu") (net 13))
 (via (at 160.511765 67.111765) (size 0.6) (drill 0.3) (layers "F.Cu" "B.Cu") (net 13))
 (segment (start 152.262 46.142) (end 148.120105 46.142) (width 0.2) (layer "B.Cu") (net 13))
 (segment (start 147.498 43.602) (end 148.56 42.54) (width 0.2) (layer "B.Cu") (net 13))
 (segment (start 147.498 45.519895) (end 147.498 43.602) (width 0.2) (layer "B.Cu") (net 13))
 (segment (start 148.120105 46.142) (end 147.498 45.519895) (width 0.2) (layer "B.Cu") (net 13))
 (segment (start 155.7 62.3) (end 155.7 49.58) (width 0.2) (layer "B.Cu") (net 13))
 (segment (start 160.511765 67.111765) (end 155.7 62.3) (width 0.2) (layer "B.Cu") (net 13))
 (segment (start 155.7 49.58) (end 152.262 46.142) (width 0.2) (layer "B.Cu") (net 13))
 (segment (start 161.175 53.875) (end 160.5 53.2) (width 0.2) (layer "F.Cu") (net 12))
 (segment (start 161.175 63.1) (end 161.175 53.875) (width 0.2) (layer "F.Cu") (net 12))
 (via (at 160.5 53.2) (size 0.6) (drill 0.3) (layers "F.Cu" "B.Cu") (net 12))
 (segment (start 152.38 45.08) (end 148.56 45.08) (width 0.2) (layer "B.Cu") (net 12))
 (segment (start 160.5 53.2) (end 152.38 45.08) (width 0.2) (layer "B.Cu") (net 12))
 (segment (start 124.74 83.02) (end 124.74 103.94) (width 0.2) (layer "F.Cu") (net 10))
 (segment (start 124.64 63.12) (end 124.64 61.564366) (width 0.2) (layer "F.Cu") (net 10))
 (segment (start 124.64 61.564366) (end 133.504366 52.7) (width 0.2) (layer "F.Cu") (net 10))
 (segment (start 124.64 63.12) (end 124.64 82.92) (width 0.2) (layer "F.Cu") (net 10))
 (segment (start 124.64 82.92) (end 124.74 83.02) (width 0.2) (layer "F.Cu") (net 10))
 (segment (start 124.74 103.94) (end 124.9 104.1) (width 0.2) (layer "F.Cu") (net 10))
 (segment (start 133.504366 52.7) (end 148.56 52.7) (width 0.2) (layer "F.Cu") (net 10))
 (segment (start 163.8 54.3) (end 163.8 52.7) (width 0.2) (layer "F.Cu") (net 1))
 (segment (start 144.25 66.725685) (end 144.25 77.420101) (width 0.2) (layer "F.Cu") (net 1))
 (segment (start 141.450101 83.02) (end 139.49 84.980101) (width 0.2) (layer "F.Cu") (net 1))
 (segment (start 139.64 86.96) (end 143.58 83.02) (width 0.2) (layer "F.Cu") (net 1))
 (segment (start 163.9 54.4) (end 163.8 54.3) (width 0.2) (layer "F.Cu") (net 1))
 (segment (start 136.62 55.4) (end 133.49 55.4) (width 0.2) (layer "F.Cu") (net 1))
 (segment (start 144.25 77.420101) (end 136.69 84.980101) (width 0.2) (layer "F.Cu") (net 1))
 (segment (start 136.69 86.139899) (end 137.510101 86.96) (width 0.2) (layer "F.Cu") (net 1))
 (segment (start 143.58 83.02) (end 144.44 83.02) (width 0.2) (layer "F.Cu") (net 1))
 (segment (start 144.44 63.22) (end 136.62 55.4) (width 0.2) (layer "F.Cu") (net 1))
 (segment (start 133.49 55.4) (end 133.49 57.6) (width 0.2) (layer "F.Cu") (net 1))
 (segment (start 144.44 63.22) (end 144.52 63.22) (width 0.2) (layer "F.Cu") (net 1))
 (segment (start 139.49 84.980101) (end 139.49 92.01) (width 0.2) (layer "F.Cu") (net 1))
 (segment (start 139.49 92.01) (end 137.3 94.2) (width 0.2) (layer "F.Cu") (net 1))
 (segment (start 154.6 53.3) (end 158.9 53.3) (width 0.2) (layer "F.Cu") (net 1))
 (segment (start 136.69 84.980101) (end 136.69 86.139899) (width 0.2) (layer "F.Cu") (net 1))
 (segment (start 144.44 83.02) (end 141.450101 83.02) (width 0.2) (layer "F.Cu") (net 1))
 (segment (start 144.6 63.3) (end 154.6 53.3) (width 0.2) (layer "F.Cu") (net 1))
 (segment (start 137.510101 86.96) (end 139.64 86.96) (width 0.2) (layer "F.Cu") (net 1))
 (segment (start 133.49 57.6) (end 135.124315 57.6) (width 0.2) (layer "F.Cu") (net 1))
 (segment (start 163.9 54.8) (end 163.9 54.4) (width 0.2) (layer "F.Cu") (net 1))
 (segment (start 144.52 63.22) (end 144.6 63.3) (width 0.2) (layer "F.Cu") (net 1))
 (segment (start 135.124315 57.6) (end 144.25 66.725685) (width 0.2) (layer "F.Cu") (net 1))
 (via (at 158.9 53.3) (size 0.6) (drill 0.3) (layers "F.Cu" "B.Cu") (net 1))
 (via (at 137.3 94.2) (size 0.6) (drill 0.3) (layers "F.Cu" "B.Cu") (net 1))
 (via (at 163.9 54.8) (size 0.6) (drill 0.3) (layers "F.Cu" "B.Cu") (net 1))
 (segment (start 137.3 95.68) (end 144.44 102.82) (width 0.2) (layer "B.Cu") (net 1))
 (segment (start 160.9 53.8) (end 161.9 54.8) (width 0.2) (layer "B.Cu") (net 1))
 (segment (start 158.9 53.3) (end 159.4 53.8) (width 0.2) (layer "B.Cu") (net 1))
 (segment (start 161.9 54.8) (end 163.9 54.8) (width 0.2) (layer "B.Cu") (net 1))
 (segment (start 159.4 53.8) (end 160.9 53.8) (width 0.2) (layer "B.Cu") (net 1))
 (segment (start 137.3 94.2) (end 137.3 95.68) (width 0.2) (layer "B.Cu") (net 1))
 (segment (start 175.4 54.825) (end 175.4 54.2) (width 0.2) (layer "F.Cu") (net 15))
 (segment (start 183.675 63.1) (end 175.4 54.825) (width 0.2) (layer "F.Cu") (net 15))
 (via (at 175.4 54.2) (size 0.6) (drill 0.3) (layers "F.Cu" "B.Cu") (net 15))
 (segment (start 162.76 54.2) (end 148.56 40) (width 0.2) (layer "B.Cu") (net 15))
 (segment (start 175.4 54.2) (end 162.76 54.2) (width 0.2) (layer "B.Cu") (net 15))
 (segment (start 184.975 55.482786) (end 165.890214 36.398) (width 0.2) (layer "F.Cu") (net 16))
 (segment (start 183.675 68.1) (end 184.975 66.8) (width 0.2) (layer "F.Cu") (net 16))
 (segment (start 165.890214 36.398) (end 149.622 36.398) (width 0.2) (layer "F.Cu") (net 16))
 (segment (start 184.975 66.8) (end 184.975 55.482786) (width 0.2) (layer "F.Cu") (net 16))
 (segment (start 149.622 36.398) (end 148.56 37.46) (width 0.2) (layer "F.Cu") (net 16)))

